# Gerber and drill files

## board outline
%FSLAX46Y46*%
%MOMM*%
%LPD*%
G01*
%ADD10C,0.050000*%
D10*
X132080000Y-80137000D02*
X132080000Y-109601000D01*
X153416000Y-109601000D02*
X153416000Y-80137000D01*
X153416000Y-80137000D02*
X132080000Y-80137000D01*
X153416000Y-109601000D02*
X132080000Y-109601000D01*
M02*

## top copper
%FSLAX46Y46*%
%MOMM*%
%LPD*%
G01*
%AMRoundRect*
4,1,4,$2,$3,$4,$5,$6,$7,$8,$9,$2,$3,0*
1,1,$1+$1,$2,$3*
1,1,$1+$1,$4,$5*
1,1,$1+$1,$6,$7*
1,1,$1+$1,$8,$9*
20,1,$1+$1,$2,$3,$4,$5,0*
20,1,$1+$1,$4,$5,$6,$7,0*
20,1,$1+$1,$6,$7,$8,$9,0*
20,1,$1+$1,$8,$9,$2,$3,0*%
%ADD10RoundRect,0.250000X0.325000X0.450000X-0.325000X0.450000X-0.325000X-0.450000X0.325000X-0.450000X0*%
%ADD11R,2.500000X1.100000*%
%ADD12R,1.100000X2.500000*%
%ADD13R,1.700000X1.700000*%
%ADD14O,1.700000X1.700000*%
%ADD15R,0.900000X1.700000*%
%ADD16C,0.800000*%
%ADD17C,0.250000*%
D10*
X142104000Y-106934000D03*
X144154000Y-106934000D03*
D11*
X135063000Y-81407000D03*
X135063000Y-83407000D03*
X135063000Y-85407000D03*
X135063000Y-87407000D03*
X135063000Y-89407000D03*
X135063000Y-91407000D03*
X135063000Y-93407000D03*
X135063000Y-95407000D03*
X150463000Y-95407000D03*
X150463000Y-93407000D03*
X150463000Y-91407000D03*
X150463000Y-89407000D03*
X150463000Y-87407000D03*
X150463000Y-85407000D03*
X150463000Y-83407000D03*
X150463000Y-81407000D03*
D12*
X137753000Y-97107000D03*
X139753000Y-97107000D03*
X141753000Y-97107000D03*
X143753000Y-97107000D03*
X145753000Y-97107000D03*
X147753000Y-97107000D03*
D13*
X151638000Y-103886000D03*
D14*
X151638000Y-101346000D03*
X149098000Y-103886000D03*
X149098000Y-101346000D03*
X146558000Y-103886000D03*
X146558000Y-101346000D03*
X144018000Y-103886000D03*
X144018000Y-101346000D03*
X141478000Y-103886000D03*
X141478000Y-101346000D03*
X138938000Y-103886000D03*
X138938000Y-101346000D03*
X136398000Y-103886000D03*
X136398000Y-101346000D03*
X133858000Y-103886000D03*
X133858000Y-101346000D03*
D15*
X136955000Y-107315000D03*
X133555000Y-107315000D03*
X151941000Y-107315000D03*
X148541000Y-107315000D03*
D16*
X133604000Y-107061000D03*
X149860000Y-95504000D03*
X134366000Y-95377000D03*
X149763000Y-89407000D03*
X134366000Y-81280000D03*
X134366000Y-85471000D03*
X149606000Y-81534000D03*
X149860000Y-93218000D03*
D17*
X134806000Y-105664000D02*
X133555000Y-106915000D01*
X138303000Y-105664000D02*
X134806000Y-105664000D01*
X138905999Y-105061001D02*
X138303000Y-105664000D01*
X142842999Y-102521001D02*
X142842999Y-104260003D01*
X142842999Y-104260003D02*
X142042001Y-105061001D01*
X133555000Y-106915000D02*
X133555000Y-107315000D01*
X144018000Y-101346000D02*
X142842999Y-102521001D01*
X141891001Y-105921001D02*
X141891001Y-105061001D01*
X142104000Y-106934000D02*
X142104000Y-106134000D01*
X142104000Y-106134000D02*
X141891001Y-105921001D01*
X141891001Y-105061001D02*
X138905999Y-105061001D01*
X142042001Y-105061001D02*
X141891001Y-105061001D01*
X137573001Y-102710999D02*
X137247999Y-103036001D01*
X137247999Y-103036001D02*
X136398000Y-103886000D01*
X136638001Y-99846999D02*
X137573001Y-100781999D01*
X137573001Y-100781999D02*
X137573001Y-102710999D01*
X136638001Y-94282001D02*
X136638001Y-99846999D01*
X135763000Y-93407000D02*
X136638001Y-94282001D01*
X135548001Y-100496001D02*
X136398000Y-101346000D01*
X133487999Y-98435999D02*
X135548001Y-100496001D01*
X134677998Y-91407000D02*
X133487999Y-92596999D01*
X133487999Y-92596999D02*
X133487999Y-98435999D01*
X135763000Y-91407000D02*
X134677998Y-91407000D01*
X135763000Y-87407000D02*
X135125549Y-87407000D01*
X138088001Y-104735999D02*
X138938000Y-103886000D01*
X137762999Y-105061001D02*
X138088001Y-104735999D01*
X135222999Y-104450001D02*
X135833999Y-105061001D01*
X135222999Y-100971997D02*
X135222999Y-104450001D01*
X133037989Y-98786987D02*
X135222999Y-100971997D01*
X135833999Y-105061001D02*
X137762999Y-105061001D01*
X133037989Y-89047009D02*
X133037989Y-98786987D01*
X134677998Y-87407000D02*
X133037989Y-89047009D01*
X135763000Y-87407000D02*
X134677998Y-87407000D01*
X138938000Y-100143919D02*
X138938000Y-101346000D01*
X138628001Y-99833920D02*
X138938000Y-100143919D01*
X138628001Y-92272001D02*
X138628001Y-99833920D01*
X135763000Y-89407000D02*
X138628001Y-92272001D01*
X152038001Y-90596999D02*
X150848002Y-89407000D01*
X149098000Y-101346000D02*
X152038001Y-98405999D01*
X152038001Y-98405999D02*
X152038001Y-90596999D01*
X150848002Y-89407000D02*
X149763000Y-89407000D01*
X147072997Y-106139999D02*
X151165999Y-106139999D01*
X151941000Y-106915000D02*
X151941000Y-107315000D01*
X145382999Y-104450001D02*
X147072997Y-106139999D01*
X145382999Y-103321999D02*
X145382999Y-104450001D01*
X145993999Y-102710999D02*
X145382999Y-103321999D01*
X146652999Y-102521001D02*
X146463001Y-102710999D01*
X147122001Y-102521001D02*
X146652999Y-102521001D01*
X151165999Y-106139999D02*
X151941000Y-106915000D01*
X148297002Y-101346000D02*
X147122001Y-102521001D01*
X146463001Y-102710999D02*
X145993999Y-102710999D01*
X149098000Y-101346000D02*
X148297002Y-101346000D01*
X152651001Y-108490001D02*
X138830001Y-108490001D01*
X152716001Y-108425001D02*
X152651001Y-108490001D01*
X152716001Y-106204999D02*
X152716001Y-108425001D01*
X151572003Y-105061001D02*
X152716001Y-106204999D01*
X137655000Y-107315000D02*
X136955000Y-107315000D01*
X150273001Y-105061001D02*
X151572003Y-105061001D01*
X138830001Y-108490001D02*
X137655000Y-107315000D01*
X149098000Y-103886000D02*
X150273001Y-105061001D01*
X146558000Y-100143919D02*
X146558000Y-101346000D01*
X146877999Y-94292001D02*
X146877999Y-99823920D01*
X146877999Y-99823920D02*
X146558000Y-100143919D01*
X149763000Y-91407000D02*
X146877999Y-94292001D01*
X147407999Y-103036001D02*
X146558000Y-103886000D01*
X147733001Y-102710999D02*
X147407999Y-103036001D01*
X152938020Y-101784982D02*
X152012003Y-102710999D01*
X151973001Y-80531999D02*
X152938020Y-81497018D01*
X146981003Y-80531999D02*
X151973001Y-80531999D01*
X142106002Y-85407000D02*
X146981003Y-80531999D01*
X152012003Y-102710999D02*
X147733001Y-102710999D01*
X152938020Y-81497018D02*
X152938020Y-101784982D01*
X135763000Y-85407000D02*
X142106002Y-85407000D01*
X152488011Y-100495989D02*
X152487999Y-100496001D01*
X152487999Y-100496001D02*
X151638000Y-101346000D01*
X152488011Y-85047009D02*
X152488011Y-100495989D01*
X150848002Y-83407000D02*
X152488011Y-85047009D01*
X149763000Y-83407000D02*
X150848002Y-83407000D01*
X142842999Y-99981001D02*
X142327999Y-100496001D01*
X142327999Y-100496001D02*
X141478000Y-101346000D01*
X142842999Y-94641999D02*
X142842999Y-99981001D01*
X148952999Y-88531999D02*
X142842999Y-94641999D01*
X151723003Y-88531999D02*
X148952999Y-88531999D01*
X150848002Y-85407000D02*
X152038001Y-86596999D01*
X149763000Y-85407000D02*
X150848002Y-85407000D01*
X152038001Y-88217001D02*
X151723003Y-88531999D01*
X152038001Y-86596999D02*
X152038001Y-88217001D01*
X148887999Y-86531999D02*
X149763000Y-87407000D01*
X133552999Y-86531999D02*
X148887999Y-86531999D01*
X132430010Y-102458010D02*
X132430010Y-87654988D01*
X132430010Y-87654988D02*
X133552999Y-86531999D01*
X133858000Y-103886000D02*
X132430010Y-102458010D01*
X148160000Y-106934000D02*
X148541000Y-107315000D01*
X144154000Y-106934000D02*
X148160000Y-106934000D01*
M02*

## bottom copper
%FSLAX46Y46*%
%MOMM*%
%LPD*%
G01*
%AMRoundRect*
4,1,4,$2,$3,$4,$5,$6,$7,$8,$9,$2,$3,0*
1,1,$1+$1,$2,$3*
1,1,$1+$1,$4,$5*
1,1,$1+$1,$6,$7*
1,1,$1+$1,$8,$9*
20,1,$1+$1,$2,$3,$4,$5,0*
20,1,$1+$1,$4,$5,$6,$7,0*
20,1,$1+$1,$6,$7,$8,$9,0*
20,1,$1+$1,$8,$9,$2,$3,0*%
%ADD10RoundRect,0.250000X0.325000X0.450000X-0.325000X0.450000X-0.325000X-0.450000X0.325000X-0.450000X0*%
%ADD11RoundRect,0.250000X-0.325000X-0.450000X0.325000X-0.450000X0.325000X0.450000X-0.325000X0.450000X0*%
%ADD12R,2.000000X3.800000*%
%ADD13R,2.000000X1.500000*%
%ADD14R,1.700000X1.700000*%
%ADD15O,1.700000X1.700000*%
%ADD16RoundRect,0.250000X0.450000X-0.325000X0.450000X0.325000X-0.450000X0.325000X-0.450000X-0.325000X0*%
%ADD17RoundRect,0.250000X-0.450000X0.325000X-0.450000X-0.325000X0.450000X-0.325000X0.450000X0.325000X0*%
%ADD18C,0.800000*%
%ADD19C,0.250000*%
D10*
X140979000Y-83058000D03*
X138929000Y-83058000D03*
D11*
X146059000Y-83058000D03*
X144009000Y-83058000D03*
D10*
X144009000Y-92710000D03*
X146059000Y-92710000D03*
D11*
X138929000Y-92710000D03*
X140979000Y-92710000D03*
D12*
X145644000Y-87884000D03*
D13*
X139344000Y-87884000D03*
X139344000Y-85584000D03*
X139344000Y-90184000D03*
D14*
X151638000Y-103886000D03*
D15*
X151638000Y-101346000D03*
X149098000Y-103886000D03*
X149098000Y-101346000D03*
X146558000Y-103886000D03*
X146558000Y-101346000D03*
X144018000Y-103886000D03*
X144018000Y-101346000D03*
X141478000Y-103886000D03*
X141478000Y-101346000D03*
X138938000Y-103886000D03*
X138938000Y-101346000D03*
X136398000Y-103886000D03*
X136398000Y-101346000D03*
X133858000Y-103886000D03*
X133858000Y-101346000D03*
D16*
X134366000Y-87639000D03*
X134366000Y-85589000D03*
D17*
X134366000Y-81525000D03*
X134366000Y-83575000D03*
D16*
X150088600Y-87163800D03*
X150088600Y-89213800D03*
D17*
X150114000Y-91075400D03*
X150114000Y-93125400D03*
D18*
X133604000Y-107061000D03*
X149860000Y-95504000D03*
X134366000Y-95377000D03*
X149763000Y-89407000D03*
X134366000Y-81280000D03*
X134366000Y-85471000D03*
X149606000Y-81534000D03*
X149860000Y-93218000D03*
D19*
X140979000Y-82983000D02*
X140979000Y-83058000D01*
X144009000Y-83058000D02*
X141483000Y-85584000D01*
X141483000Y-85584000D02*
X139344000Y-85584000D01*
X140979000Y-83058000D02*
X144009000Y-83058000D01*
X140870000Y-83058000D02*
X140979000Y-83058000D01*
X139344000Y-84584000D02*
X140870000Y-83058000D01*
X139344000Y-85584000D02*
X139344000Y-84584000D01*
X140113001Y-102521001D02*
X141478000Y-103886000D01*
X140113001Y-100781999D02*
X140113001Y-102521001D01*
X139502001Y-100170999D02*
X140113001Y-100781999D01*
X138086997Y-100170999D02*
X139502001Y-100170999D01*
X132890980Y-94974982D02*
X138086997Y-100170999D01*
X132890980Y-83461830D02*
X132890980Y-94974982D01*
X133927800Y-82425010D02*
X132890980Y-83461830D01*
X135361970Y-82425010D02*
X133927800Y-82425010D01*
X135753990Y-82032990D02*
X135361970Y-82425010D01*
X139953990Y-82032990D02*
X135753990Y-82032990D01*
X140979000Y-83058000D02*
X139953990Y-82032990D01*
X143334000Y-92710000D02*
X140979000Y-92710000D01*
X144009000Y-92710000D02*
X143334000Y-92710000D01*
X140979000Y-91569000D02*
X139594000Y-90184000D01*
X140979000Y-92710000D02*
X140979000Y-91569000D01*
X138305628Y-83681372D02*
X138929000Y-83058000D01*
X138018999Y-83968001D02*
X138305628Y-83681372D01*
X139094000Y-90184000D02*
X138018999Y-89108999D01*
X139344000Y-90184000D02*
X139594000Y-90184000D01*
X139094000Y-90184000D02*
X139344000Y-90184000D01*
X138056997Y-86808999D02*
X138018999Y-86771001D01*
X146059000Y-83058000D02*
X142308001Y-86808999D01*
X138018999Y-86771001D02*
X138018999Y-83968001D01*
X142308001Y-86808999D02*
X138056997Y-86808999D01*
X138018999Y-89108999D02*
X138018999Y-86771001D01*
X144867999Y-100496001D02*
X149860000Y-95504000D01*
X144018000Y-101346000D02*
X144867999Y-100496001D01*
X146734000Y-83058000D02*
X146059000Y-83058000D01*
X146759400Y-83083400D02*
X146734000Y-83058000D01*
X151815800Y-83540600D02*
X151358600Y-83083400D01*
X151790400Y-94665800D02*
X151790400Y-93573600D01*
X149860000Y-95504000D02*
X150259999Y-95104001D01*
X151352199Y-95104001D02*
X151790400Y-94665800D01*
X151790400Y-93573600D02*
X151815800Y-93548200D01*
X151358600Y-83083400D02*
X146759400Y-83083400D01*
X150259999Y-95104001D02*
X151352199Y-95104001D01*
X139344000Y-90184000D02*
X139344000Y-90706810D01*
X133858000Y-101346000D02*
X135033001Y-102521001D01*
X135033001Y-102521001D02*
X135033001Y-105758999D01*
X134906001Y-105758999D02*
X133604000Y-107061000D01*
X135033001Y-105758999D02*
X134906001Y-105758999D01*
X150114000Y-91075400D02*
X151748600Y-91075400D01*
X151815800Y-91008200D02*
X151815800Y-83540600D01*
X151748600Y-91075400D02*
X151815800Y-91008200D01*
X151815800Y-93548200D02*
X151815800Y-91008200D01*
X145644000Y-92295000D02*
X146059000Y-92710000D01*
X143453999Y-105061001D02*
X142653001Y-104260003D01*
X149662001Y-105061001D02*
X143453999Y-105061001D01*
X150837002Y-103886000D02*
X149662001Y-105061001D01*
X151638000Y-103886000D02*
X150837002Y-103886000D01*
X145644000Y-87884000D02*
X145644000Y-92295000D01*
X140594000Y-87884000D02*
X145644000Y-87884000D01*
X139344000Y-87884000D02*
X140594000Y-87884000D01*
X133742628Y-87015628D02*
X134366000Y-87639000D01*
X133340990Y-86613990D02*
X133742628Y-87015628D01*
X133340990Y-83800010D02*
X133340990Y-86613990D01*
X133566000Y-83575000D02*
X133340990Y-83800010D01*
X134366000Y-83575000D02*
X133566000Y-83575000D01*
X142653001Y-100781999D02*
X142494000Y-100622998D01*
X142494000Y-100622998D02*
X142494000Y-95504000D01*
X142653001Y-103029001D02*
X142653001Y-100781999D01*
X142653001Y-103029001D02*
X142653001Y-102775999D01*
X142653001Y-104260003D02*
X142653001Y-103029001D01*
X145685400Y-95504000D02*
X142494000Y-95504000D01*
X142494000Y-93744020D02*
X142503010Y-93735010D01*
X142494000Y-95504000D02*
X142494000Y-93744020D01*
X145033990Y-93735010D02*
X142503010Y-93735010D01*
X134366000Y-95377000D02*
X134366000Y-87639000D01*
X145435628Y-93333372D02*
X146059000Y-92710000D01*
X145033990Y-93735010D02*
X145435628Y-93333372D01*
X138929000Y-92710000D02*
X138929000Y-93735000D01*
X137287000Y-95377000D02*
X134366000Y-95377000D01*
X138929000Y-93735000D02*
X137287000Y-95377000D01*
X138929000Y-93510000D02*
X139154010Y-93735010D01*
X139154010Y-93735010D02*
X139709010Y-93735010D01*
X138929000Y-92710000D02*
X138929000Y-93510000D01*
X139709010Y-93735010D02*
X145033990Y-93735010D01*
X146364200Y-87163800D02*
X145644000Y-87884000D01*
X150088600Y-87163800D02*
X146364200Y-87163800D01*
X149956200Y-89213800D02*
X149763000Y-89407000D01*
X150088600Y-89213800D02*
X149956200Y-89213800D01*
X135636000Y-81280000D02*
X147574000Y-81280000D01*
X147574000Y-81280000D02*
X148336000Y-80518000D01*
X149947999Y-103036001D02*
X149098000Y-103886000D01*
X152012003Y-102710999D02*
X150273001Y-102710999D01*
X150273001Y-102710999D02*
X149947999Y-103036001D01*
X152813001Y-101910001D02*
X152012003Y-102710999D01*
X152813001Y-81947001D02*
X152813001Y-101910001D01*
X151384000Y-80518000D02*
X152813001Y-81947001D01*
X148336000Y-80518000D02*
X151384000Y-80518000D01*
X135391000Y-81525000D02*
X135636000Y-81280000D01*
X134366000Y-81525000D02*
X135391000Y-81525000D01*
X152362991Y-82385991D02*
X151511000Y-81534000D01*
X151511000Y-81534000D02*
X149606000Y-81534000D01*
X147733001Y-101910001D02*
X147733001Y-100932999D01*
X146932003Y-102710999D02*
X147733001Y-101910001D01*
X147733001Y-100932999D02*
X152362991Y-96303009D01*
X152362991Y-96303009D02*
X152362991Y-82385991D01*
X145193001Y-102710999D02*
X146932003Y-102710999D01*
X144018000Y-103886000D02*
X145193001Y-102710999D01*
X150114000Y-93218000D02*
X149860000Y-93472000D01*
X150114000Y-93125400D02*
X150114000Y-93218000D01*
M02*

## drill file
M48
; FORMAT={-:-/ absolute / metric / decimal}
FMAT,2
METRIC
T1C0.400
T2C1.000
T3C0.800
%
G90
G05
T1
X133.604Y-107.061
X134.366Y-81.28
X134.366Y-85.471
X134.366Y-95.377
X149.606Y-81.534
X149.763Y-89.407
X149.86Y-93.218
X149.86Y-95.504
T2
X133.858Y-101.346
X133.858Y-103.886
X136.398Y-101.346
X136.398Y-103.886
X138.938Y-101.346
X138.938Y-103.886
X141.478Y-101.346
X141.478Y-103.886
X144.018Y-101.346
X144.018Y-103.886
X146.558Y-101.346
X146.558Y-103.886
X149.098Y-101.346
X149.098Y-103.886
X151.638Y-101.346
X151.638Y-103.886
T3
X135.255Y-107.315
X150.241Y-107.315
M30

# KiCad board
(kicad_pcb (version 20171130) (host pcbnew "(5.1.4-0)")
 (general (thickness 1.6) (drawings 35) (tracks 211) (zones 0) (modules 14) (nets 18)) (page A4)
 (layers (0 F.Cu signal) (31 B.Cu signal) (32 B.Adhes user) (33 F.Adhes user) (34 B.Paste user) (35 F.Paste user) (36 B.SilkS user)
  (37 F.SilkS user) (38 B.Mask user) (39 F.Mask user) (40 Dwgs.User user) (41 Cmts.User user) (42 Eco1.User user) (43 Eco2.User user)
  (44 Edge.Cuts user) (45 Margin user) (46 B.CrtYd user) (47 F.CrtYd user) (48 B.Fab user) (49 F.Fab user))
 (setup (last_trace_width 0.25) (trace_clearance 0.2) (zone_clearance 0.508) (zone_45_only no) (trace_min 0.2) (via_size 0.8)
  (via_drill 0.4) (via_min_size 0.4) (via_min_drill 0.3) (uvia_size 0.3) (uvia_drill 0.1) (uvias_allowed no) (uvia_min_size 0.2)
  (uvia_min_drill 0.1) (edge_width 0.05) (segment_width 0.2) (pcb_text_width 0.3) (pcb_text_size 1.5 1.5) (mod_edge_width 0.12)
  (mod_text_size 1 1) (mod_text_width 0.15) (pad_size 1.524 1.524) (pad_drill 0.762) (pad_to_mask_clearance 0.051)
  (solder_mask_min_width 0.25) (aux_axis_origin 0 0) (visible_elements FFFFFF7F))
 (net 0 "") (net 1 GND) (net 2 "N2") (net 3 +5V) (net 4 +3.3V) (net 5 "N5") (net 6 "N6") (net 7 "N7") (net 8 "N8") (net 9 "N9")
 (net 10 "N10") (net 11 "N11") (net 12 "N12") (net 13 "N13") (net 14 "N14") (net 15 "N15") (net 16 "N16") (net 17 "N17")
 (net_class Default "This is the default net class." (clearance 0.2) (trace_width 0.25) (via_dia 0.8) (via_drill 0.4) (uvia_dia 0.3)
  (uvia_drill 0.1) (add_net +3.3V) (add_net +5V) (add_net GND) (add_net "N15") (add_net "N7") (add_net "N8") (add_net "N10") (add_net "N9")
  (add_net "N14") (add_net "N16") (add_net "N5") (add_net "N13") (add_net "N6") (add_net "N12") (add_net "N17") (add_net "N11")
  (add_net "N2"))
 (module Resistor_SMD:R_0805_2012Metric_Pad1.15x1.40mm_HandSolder (layer F.Cu) (at 143.129 106.934 180)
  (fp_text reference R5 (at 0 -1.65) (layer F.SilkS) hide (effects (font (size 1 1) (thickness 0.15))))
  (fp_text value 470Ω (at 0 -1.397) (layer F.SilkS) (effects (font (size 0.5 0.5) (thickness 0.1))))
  (pad 2 smd roundrect (at 1.025 0 180) (size 1.15 1.4) (layers F.Cu F.Paste F.Mask) (roundrect_rratio 0.217391) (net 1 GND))
  (pad 1 smd roundrect (at -1.025 0 180) (size 1.15 1.4) (layers F.Cu F.Paste F.Mask) (roundrect_rratio 0.217391) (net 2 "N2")))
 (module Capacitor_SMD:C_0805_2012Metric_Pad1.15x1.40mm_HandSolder (layer B.Cu) (at 139.954 83.058 180)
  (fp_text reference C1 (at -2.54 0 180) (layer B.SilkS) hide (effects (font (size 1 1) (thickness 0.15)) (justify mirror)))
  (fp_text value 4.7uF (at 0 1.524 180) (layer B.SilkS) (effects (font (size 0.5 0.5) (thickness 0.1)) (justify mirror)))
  (pad 1 smd roundrect (at -1.025 0 180) (size 1.15 1.4) (layers B.Cu B.Paste B.Mask) (roundrect_rratio 0.217391) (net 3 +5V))
  (pad 2 smd roundrect (at 1.025 0 180) (size 1.15 1.4) (layers B.Cu B.Paste B.Mask) (roundrect_rratio 0.217391) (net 1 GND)))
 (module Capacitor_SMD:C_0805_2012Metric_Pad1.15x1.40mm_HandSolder (layer B.Cu) (at 145.034 83.058)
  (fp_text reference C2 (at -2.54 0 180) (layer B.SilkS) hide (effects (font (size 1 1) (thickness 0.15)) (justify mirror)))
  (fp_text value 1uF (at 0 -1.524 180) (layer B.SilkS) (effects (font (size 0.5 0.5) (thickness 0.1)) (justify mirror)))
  (pad 2 smd roundrect (at 1.025 0) (size 1.15 1.4) (layers B.Cu B.Paste B.Mask) (roundrect_rratio 0.217391) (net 1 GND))
  (pad 1 smd roundrect (at -1.025 0) (size 1.15 1.4) (layers B.Cu B.Paste B.Mask) (roundrect_rratio 0.217391) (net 3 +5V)))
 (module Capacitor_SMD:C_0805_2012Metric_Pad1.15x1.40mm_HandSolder (layer B.Cu) (at 145.034 92.71 180)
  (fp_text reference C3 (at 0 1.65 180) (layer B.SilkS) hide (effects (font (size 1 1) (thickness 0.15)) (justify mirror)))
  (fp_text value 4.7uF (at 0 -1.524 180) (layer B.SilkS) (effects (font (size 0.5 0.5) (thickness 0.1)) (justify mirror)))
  (pad 2 smd roundrect (at 1.025 0 180) (size 1.15 1.4) (layers B.Cu B.Paste B.Mask) (roundrect_rratio 0.217391) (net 1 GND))
  (pad 1 smd roundrect (at -1.025 0 180) (size 1.15 1.4) (layers B.Cu B.Paste B.Mask) (roundrect_rratio 0.217391) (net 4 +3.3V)))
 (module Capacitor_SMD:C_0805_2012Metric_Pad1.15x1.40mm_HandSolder (layer B.Cu) (at 139.954 92.71)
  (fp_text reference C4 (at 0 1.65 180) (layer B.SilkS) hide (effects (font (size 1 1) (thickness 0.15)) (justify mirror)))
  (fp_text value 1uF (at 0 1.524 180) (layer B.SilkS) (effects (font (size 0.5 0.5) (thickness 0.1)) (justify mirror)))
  (pad 1 smd roundrect (at -1.025 0) (size 1.15 1.4) (layers B.Cu B.Paste B.Mask) (roundrect_rratio 0.217391) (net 4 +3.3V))
  (pad 2 smd roundrect (at 1.025 0) (size 1.15 1.4) (layers B.Cu B.Paste B.Mask) (roundrect_rratio 0.217391) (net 1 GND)))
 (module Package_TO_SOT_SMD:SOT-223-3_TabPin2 (layer B.Cu) (at 142.494 87.884)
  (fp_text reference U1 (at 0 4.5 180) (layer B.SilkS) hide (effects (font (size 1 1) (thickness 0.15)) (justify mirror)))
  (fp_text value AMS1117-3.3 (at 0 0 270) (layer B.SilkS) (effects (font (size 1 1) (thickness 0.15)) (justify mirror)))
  (pad 2 smd rect (at 3.15 0) (size 2 3.8) (layers B.Cu B.Paste B.Mask) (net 4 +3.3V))
  (pad 2 smd rect (at -3.15 0) (size 2 1.5) (layers B.Cu B.Paste B.Mask) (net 4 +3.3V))
  (pad 3 smd rect (at -3.15 -2.3) (size 2 1.5) (layers B.Cu B.Paste B.Mask) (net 3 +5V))
  (pad 1 smd rect (at -3.15 2.3) (size 2 1.5) (layers B.Cu B.Paste B.Mask) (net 1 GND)))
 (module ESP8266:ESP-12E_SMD (layer F.Cu) (at 135.763 81.407)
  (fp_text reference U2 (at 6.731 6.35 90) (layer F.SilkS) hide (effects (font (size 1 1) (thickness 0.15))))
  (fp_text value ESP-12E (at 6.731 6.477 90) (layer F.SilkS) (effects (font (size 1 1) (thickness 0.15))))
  (pad 1 smd rect (at 0 0) (size 2.5 1.1) (drill (offset -0.7 0)) (layers F.Cu F.Paste F.Mask) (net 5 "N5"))
  (pad 2 smd rect (at 0 2) (size 2.5 1.1) (drill (offset -0.7 0)) (layers F.Cu F.Paste F.Mask))
  (pad 3 smd rect (at 0 4) (size 2.5 1.1) (drill (offset -0.7 0)) (layers F.Cu F.Paste F.Mask) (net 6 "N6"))
  (pad 4 smd rect (at 0 6) (size 2.5 1.1) (drill (offset -0.7 0)) (layers F.Cu F.Paste F.Mask) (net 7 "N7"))
  (pad 5 smd rect (at 0 8) (size 2.5 1.1) (drill (offset -0.7 0)) (layers F.Cu F.Paste F.Mask) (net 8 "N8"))
  (pad 6 smd rect (at 0 10) (size 2.5 1.1) (drill (offset -0.7 0)) (layers F.Cu F.Paste F.Mask) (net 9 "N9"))
  (pad 7 smd rect (at 0 12) (size 2.5 1.1) (drill (offset -0.7 0)) (layers F.Cu F.Paste F.Mask) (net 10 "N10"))
  (pad 8 smd rect (at 0 14) (size 2.5 1.1) (drill (offset -0.7 0)) (layers F.Cu F.Paste F.Mask) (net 4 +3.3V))
  (pad 9 smd rect (at 14 14) (size 2.5 1.1) (drill (offset 0.7 0)) (layers F.Cu F.Paste F.Mask) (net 1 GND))
  (pad 10 smd rect (at 14 12) (size 2.5 1.1) (drill (offset 0.7 0)) (layers F.Cu F.Paste F.Mask) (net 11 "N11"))
  (pad 11 smd rect (at 14 10) (size 2.5 1.1) (drill (offset 0.7 0)) (layers F.Cu F.Paste F.Mask) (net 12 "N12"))
  (pad 12 smd rect (at 14 8) (size 2.5 1.1) (drill (offset 0.7 0)) (layers F.Cu F.Paste F.Mask) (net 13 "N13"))
  (pad 13 smd rect (at 14 6) (size 2.5 1.1) (drill (offset 0.7 0)) (layers F.Cu F.Paste F.Mask) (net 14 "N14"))
  (pad 14 smd rect (at 14 4) (size 2.5 1.1) (drill (offset 0.7 0)) (layers F.Cu F.Paste F.Mask) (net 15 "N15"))
  (pad 15 smd rect (at 14 2) (size 2.5 1.1) (drill (offset 0.7 0)) (layers F.Cu F.Paste F.Mask) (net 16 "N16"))
  (pad 16 smd rect (at 14 0) (size 2.5 1.1) (drill (offset 0.7 0)) (layers F.Cu F.Paste F.Mask) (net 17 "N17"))
  (pad 17 smd rect (at 1.99 15 90) (size 2.5 1.1) (drill (offset -0.7 0)) (layers F.Cu F.Paste F.Mask))
  (pad 18 smd rect (at 3.99 15 90) (size 2.5 1.1) (drill (offset -0.7 0)) (layers F.Cu F.Paste F.Mask))
  (pad 19 smd rect (at 5.99 15 90) (size 2.5 1.1) (drill (offset -0.7 0)) (layers F.Cu F.Paste F.Mask))
  (pad 20 smd rect (at 7.99 15 90) (size 2.5 1.1) (drill (offset -0.7 0)) (layers F.Cu F.Paste F.Mask))
  (pad 21 smd rect (at 9.99 15 90) (size 2.5 1.1) (drill (offset -0.7 0)) (layers F.Cu F.Paste F.Mask))
  (pad 22 smd rect (at 11.99 15 90) (size 2.5 1.1) (drill (offset -0.7 0)) (layers F.Cu F.Paste F.Mask)))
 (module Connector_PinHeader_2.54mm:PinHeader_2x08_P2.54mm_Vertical (layer B.Cu) (at 151.638 103.886 90)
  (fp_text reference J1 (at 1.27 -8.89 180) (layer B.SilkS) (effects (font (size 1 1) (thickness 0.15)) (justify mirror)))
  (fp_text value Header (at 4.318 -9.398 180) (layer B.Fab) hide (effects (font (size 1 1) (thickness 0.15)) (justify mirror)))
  (pad 1 thru_hole rect (at 0 0 90) (size 1.7 1.7) (drill 1) (layers *.Cu *.Mask) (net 4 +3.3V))
  (pad 2 thru_hole oval (at 2.54 0 90) (size 1.7 1.7) (drill 1) (layers *.Cu *.Mask) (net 16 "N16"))
  (pad 3 thru_hole oval (at 0 -2.54 90) (size 1.7 1.7) (drill 1) (layers *.Cu *.Mask) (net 5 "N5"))
  (pad 4 thru_hole oval (at 2.54 -2.54 90) (size 1.7 1.7) (drill 1) (layers *.Cu *.Mask) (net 13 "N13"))
  (pad 5 thru_hole oval (at 0 -5.08 90) (size 1.7 1.7) (drill 1) (layers *.Cu *.Mask) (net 6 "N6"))
  (pad 6 thru_hole oval (at 2.54 -5.08 90) (size 1.7 1.7) (drill 1) (layers *.Cu *.Mask) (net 12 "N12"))
  (pad 7 thru_hole oval (at 0 -7.62 90) (size 1.7 1.7) (drill 1) (layers *.Cu *.Mask) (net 17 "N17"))
  (pad 8 thru_hole oval (at 2.54 -7.62 90) (size 1.7 1.7) (drill 1) (layers *.Cu *.Mask) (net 1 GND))
  (pad 9 thru_hole oval (at 0 -10.16 90) (size 1.7 1.7) (drill 1) (layers *.Cu *.Mask) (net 3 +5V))
  (pad 10 thru_hole oval (at 2.54 -10.16 90) (size 1.7 1.7) (drill 1) (layers *.Cu *.Mask) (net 15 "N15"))
  (pad 11 thru_hole oval (at 0 -12.7 90) (size 1.7 1.7) (drill 1) (layers *.Cu *.Mask) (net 7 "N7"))
  (pad 12 thru_hole oval (at 2.54 -12.7 90) (size 1.7 1.7) (drill 1) (layers *.Cu *.Mask) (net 8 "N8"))
  (pad 13 thru_hole oval (at 0 -15.24 90) (size 1.7 1.7) (drill 1) (layers *.Cu *.Mask) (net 10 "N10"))
  (pad 14 thru_hole oval (at 2.54 -15.24 90) (size 1.7 1.7) (drill 1) (layers *.Cu *.Mask) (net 9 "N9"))
  (pad 15 thru_hole oval (at 0 -17.78 90) (size 1.7 1.7) (drill 1) (layers *.Cu *.Mask) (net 14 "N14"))
  (pad 16 thru_hole oval (at 2.54 -17.78 90) (size 1.7 1.7) (drill 1) (layers *.Cu *.Mask) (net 1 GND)))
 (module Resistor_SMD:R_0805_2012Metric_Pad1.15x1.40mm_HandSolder (layer B.Cu) (at 134.366 86.614 90)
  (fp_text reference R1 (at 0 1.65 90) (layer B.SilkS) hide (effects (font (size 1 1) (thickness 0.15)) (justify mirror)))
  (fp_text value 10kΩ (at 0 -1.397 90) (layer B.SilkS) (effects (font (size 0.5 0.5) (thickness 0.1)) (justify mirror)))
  (pad 1 smd roundrect (at -1.025 0 90) (size 1.15 1.4) (layers B.Cu B.Paste B.Mask) (roundrect_rratio 0.217391) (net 4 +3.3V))
  (pad 2 smd roundrect (at 1.025 0 90) (size 1.15 1.4) (layers B.Cu B.Paste B.Mask) (roundrect_rratio 0.217391) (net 6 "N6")))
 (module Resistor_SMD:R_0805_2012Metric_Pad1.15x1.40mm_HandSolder (layer B.Cu) (at 134.366 82.55 270)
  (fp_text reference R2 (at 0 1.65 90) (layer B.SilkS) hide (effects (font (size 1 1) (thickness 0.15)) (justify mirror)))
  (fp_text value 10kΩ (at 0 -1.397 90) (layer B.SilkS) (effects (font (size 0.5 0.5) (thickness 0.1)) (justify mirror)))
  (pad 1 smd roundrect (at -1.025 0 270) (size 1.15 1.4) (layers B.Cu B.Paste B.Mask) (roundrect_rratio 0.217391) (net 5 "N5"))
  (pad 2 smd roundrect (at 1.025 0 270) (size 1.15 1.4) (layers B.Cu B.Paste B.Mask) (roundrect_rratio 0.217391) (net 4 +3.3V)))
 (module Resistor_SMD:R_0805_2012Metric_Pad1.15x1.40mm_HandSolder (layer B.Cu) (at 150.0886 88.1888 90)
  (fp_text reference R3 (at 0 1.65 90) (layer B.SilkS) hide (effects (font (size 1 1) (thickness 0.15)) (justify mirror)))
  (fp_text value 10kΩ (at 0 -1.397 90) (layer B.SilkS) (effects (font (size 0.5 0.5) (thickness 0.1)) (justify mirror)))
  (pad 2 smd roundrect (at 1.025 0 90) (size 1.15 1.4) (layers B.Cu B.Paste B.Mask) (roundrect_rratio 0.217391) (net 4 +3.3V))
  (pad 1 smd roundrect (at -1.025 0 90) (size 1.15 1.4) (layers B.Cu B.Paste B.Mask) (roundrect_rratio 0.217391) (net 13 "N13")))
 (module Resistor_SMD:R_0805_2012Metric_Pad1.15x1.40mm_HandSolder (layer B.Cu) (at 150.114 92.1004 270)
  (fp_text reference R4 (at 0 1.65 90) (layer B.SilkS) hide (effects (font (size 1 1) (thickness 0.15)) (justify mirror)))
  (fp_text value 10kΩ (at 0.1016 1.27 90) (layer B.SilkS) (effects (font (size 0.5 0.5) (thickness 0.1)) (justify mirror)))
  (pad 1 smd roundrect (at -1.025 0 270) (size 1.15 1.4) (layers B.Cu B.Paste B.Mask) (roundrect_rratio 0.217391) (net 1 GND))
  (pad 2 smd roundrect (at 1.025 0 270) (size 1.15 1.4) (layers B.Cu B.Paste B.Mask) (roundrect_rratio 0.217391) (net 11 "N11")))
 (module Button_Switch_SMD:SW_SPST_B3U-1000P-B (layer F.Cu) (at 135.255 107.315)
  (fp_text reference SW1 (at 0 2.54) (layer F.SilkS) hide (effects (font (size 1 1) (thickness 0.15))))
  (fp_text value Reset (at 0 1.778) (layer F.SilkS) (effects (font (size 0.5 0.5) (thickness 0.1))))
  (pad "" np_thru_hole circle (at 0 0) (size 0.8 0.8) (drill 0.8) (layers *.Cu *.Mask))
  (pad 2 smd rect (at 1.7 0) (size 0.9 1.7) (layers F.Cu F.Paste F.Mask) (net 5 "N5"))
  (pad 1 smd rect (at -1.7 0) (size 0.9 1.7) (layers F.Cu F.Paste F.Mask) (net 1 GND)))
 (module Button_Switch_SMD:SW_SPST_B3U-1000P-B (layer F.Cu) (at 150.241 107.315 180)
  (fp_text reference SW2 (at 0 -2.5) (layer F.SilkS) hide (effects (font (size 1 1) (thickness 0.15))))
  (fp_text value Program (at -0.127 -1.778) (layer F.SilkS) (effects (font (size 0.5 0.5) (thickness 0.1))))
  (pad 1 smd rect (at -1.7 0 180) (size 0.9 1.7) (layers F.Cu F.Paste F.Mask) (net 13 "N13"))
  (pad 2 smd rect (at 1.7 0 180) (size 0.9 1.7) (layers F.Cu F.Paste F.Mask) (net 2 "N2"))
  (pad "" np_thru_hole circle (at 0 0 180) (size 0.8 0.8) (drill 0.8) (layers *.Cu *.Mask)))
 (gr_line (start 132.08 80.137) (end 132.08 109.601) (layer Edge.Cuts) (width 0.05))
 (gr_line (start 153.416 109.601) (end 153.416 80.137) (layer Edge.Cuts) (width 0.05))
 (gr_line (start 153.416 80.137) (end 132.08 80.137) (layer Edge.Cuts) (width 0.05))
 (gr_line (start 153.416 109.601) (end 132.08 109.601) (layer Edge.Cuts) (width 0.05))
 (segment (start 140.979 82.983) (end 140.979 83.058) (width 0.25) (layer B.Cu) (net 3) (status 30))
 (segment (start 144.009 83.058) (end 141.483 85.584) (width 0.25) (layer B.Cu) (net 3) (status 10))
 (segment (start 141.483 85.584) (end 139.344 85.584) (width 0.25) (layer B.Cu) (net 3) (status 20))
 (segment (start 140.979 83.058) (end 144.009 83.058) (width 0.25) (layer B.Cu) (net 3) (status 30))
 (segment (start 140.87 83.058) (end 140.979 83.058) (width 0.25) (layer B.Cu) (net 3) (status 30))
 (segment (start 139.344 84.584) (end 140.87 83.058) (width 0.25) (layer B.Cu) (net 3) (status 20))
 (segment (start 139.344 85.584) (end 139.344 84.584) (width 0.25) (layer B.Cu) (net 3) (status 10))
 (segment (start 140.113001 102.521001) (end 141.478 103.886) (width 0.25) (layer B.Cu) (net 3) (status 20))
 (segment (start 140.113001 100.781999) (end 140.113001 102.521001) (width 0.25) (layer B.Cu) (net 3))
 (segment (start 139.502001 100.170999) (end 140.113001 100.781999) (width 0.25) (layer B.Cu) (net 3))
 (segment (start 138.086997 100.170999) (end 139.502001 100.170999) (width 0.25) (layer B.Cu) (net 3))
 (segment (start 132.89098 94.974982) (end 138.086997 100.170999) (width 0.25) (layer B.Cu) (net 3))
 (segment (start 132.89098 83.46183) (end 132.89098 94.974982) (width 0.25) (layer B.Cu) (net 3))
 (segment (start 133.9278 82.42501) (end 132.89098 83.46183) (width 0.25) (layer B.Cu) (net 3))
 (segment (start 135.36197 82.42501) (end 133.9278 82.42501) (width 0.25) (layer B.Cu) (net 3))
 (segment (start 135.75399 82.03299) (end 135.36197 82.42501) (width 0.25) (layer B.Cu) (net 3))
 (segment (start 139.95399 82.03299) (end 135.75399 82.03299) (width 0.25) (layer B.Cu) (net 3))
 (segment (start 140.979 83.058) (end 139.95399 82.03299) (width 0.25) (layer B.Cu) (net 3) (status 10))
 (via (at 133.604 107.061) (size 0.8) (drill 0.4) (layers F.Cu B.Cu) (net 1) (status 30))
 (via (at 149.86 95.504) (size 0.8) (drill 0.4) (layers F.Cu B.Cu) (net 1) (status 30))
 (segment (start 143.334 92.71) (end 140.979 92.71) (width 0.25) (layer B.Cu) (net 1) (status 20))
 (segment (start 144.009 92.71) (end 143.334 92.71) (width 0.25) (layer B.Cu) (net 1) (status 10))
 (segment (start 140.979 91.569) (end 139.594 90.184) (width 0.25) (layer B.Cu) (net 1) (status 20))
 (segment (start 140.979 92.71) (end 140.979 91.569) (width 0.25) (layer B.Cu) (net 1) (status 10))
 (segment (start 138.305628 83.681372) (end 138.929 83.058) (width 0.25) (layer B.Cu) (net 1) (status 20))
 (segment (start 138.018999 83.968001) (end 138.305628 83.681372) (width 0.25) (layer B.Cu) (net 1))
 (segment (start 139.094 90.184) (end 138.018999 89.108999) (width 0.25) (layer B.Cu) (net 1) (status 10))
 (segment (start 139.344 90.184) (end 139.594 90.184) (width 0.25) (layer B.Cu) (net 1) (status 30))
 (segment (start 139.094 90.184) (end 139.344 90.184) (width 0.25) (layer B.Cu) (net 1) (status 30))
 (segment (start 138.056997 86.808999) (end 138.018999 86.771001) (width 0.25) (layer B.Cu) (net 1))
 (segment (start 146.059 83.058) (end 142.308001 86.808999) (width 0.25) (layer B.Cu) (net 1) (status 10))
 (segment (start 138.018999 86.771001) (end 138.018999 83.968001) (width 0.25) (layer B.Cu) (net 1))
 (segment (start 142.308001 86.808999) (end 138.056997 86.808999) (width 0.25) (layer B.Cu) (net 1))
 (segment (start 138.018999 89.108999) (end 138.018999 86.771001) (width 0.25) (layer B.Cu) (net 1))
 (segment (start 144.867999 100.496001) (end 149.86 95.504) (width 0.25) (layer B.Cu) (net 1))
 (segment (start 144.018 101.346) (end 144.867999 100.496001) (width 0.25) (layer B.Cu) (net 1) (status 10))
 (segment (start 146.734 83.058) (end 146.059 83.058) (width 0.25) (layer B.Cu) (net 1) (status 20))
 (segment (start 146.7594 83.0834) (end 146.734 83.058) (width 0.25) (layer B.Cu) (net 1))
 (segment (start 151.8158 83.5406) (end 151.3586 83.0834) (width 0.25) (layer B.Cu) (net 1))
 (segment (start 151.7904 94.6658) (end 151.7904 93.5736) (width 0.25) (layer B.Cu) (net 1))
 (segment (start 149.86 95.504) (end 150.259999 95.104001) (width 0.25) (layer B.Cu) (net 1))
 (segment (start 151.352199 95.104001) (end 151.7904 94.6658) (width 0.25) (layer B.Cu) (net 1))
 (segment (start 151.7904 93.5736) (end 151.8158 93.5482) (width 0.25) (layer B.Cu) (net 1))
 (segment (start 151.3586 83.0834) (end 146.7594 83.0834) (width 0.25) (layer B.Cu) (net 1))
 (segment (start 150.259999 95.104001) (end 151.352199 95.104001) (width 0.25) (layer B.Cu) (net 1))
 (segment (start 139.344 90.184) (end 139.344 90.70681) (width 0.25) (layer B.Cu) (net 1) (status 30))
 (segment (start 133.858 101.346) (end 135.033001 102.521001) (width 0.25) (layer B.Cu) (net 1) (status 10))
 (segment (start 135.033001 102.521001) (end 135.033001 105.758999) (width 0.25) (layer B.Cu) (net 1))
 (segment (start 134.906001 105.758999) (end 133.604 107.061) (width 0.25) (layer B.Cu) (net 1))
 (segment (start 135.033001 105.758999) (end 134.906001 105.758999) (width 0.25) (layer B.Cu) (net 1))
 (segment (start 134.806 105.664) (end 133.555 106.915) (width 0.25) (layer F.Cu) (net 1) (status 20))
 (segment (start 138.303 105.664) (end 134.806 105.664) (width 0.25) (layer F.Cu) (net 1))
 (segment (start 138.905999 105.061001) (end 138.303 105.664) (width 0.25) (layer F.Cu) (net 1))
 (segment (start 142.842999 102.521001) (end 142.842999 104.260003) (width 0.25) (layer F.Cu) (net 1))
 (segment (start 142.842999 104.260003) (end 142.042001 105.061001) (width 0.25) (layer F.Cu) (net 1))
 (segment (start 133.555 106.915) (end 133.555 107.315) (width 0.25) (layer F.Cu) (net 1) (status 30))
 (segment (start 144.018 101.346) (end 142.842999 102.521001) (width 0.25) (layer F.Cu) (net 1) (status 10))
 (segment (start 141.891001 105.921001) (end 141.891001 105.061001) (width 0.25) (layer F.Cu) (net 1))
 (segment (start 142.104 106.934) (end 142.104 106.134) (width 0.25) (layer F.Cu) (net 1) (status 10))
 (segment (start 142.104 106.134) (end 141.891001 105.921001) (width 0.25) (layer F.Cu) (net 1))
 (segment (start 141.891001 105.061001) (end 138.905999 105.061001) (width 0.25) (layer F.Cu) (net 1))
 (segment (start 142.042001 105.061001) (end 141.891001 105.061001) (width 0.25) (layer F.Cu) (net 1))
 (segment (start 150.114 91.0754) (end 151.7486 91.0754) (width 0.25) (layer B.Cu) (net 1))
 (segment (start 151.8158 91.0082) (end 151.8158 83.5406) (width 0.25) (layer B.Cu) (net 1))
 (segment (start 151.7486 91.0754) (end 151.8158 91.0082) (width 0.25) (layer B.Cu) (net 1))
 (segment (start 151.8158 93.5482) (end 151.8158 91.0082) (width 0.25) (layer B.Cu) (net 1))
 (via (at 134.366 95.377) (size 0.8) (drill 0.4) (layers F.Cu B.Cu) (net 4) (status 30))
 (segment (start 145.644 92.295) (end 146.059 92.71) (width 0.25) (layer B.Cu) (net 4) (status 30))
 (segment (start 143.453999 105.061001) (end 142.653001 104.260003) (width 0.25) (layer B.Cu) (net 4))
 (segment (start 149.662001 105.061001) (end 143.453999 105.061001) (width 0.25) (layer B.Cu) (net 4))
 (segment (start 150.837002 103.886) (end 149.662001 105.061001) (width 0.25) (layer B.Cu) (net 4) (status 10))
 (segment (start 151.638 103.886) (end 150.837002 103.886) (width 0.25) (layer B.Cu) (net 4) (status 30))
 (segment (start 145.644 87.884) (end 145.644 92.295) (width 0.25) (layer B.Cu) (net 4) (status 30))
 (segment (start 140.594 87.884) (end 145.644 87.884) (width 0.25) (layer B.Cu) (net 4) (status 20))
 (segment (start 139.344 87.884) (end 140.594 87.884) (width 0.25) (layer B.Cu) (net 4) (status 10))
 (segment (start 133.742628 87.015628) (end 134.366 87.639) (width 0.25) (layer B.Cu) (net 4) (status 20))
 (segment (start 133.34099 86.61399) (end 133.742628 87.015628) (width 0.25) (layer B.Cu) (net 4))
 (segment (start 133.34099 83.80001) (end 133.34099 86.61399) (width 0.25) (layer B.Cu) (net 4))
 (segment (start 133.566 83.575) (end 133.34099 83.80001) (width 0.25) (layer B.Cu) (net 4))
 (segment (start 134.366 83.575) (end 133.566 83.575) (width 0.25) (layer B.Cu) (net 4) (status 10))
 (segment (start 142.653001 100.781999) (end 142.494 100.622998) (width 0.25) (layer B.Cu) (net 4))
 (segment (start 142.494 100.622998) (end 142.494 95.504) (width 0.25) (layer B.Cu) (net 4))
 (segment (start 142.653001 103.029001) (end 142.653001 100.781999) (width 0.25) (layer B.Cu) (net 4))
 (segment (start 142.653001 103.029001) (end 142.653001 102.775999) (width 0.25) (layer B.Cu) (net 4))
 (segment (start 142.653001 104.260003) (end 142.653001 103.029001) (width 0.25) (layer B.Cu) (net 4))
 (segment (start 145.6854 95.504) (end 142.494 95.504) (width 0.25) (layer B.Cu) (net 4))
 (segment (start 142.494 93.74402) (end 142.50301 93.73501) (width 0.25) (layer B.Cu) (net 4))
 (segment (start 142.494 95.504) (end 142.494 93.74402) (width 0.25) (layer B.Cu) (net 4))
 (segment (start 145.03399 93.73501) (end 142.50301 93.73501) (width 0.25) (layer B.Cu) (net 4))
 (segment (start 134.366 95.377) (end 134.366 87.639) (width 0.25) (layer B.Cu) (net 4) (status 20))
 (segment (start 145.435628 93.333372) (end 146.059 92.71) (width 0.25) (layer B.Cu) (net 4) (status 20))
 (segment (start 145.03399 93.73501) (end 145.435628 93.333372) (width 0.25) (layer B.Cu) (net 4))
 (segment (start 138.929 92.71) (end 138.929 93.735) (width 0.25) (layer B.Cu) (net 4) (status 10))
 (segment (start 137.287 95.377) (end 134.366 95.377) (width 0.25) (layer B.Cu) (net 4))
 (segment (start 138.929 93.735) (end 137.287 95.377) (width 0.25) (layer B.Cu) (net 4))
 (segment (start 138.929 93.51) (end 139.15401 93.73501) (width 0.25) (layer B.Cu) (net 4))
 (segment (start 139.15401 93.73501) (end 139.70901 93.73501) (width 0.25) (layer B.Cu) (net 4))
 (segment (start 138.929 92.71) (end 138.929 93.51) (width 0.25) (layer B.Cu) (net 4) (status 10))
 (segment (start 139.70901 93.73501) (end 145.03399 93.73501) (width 0.25) (layer B.Cu) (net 4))
 (segment (start 146.3642 87.1638) (end 145.644 87.884) (width 0.25) (layer B.Cu) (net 4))
 (segment (start 150.0886 87.1638) (end 146.3642 87.1638) (width 0.25) (layer B.Cu) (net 4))
 (segment (start 137.573001 102.710999) (end 137.247999 103.036001) (width 0.25) (layer F.Cu) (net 10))
 (segment (start 137.247999 103.036001) (end 136.398 103.886) (width 0.25) (layer F.Cu) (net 10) (status 20))
 (segment (start 136.638001 99.846999) (end 137.573001 100.781999) (width 0.25) (layer F.Cu) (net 10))
 (segment (start 137.573001 100.781999) (end 137.573001 102.710999) (width 0.25) (layer F.Cu) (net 10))
 (segment (start 136.638001 94.282001) (end 136.638001 99.846999) (width 0.25) (layer F.Cu) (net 10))
 (segment (start 135.763 93.407) (end 136.638001 94.282001) (width 0.25) (layer F.Cu) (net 10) (status 10))
 (segment (start 135.548001 100.496001) (end 136.398 101.346) (width 0.25) (layer F.Cu) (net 9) (status 20))
 (segment (start 133.487999 98.435999) (end 135.548001 100.496001) (width 0.25) (layer F.Cu) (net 9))
 (segment (start 134.677998 91.407) (end 133.487999 92.596999) (width 0.25) (layer F.Cu) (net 9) (status 10))
 (segment (start 133.487999 92.596999) (end 133.487999 98.435999) (width 0.25) (layer F.Cu) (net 9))
 (segment (start 135.763 91.407) (end 134.677998 91.407) (width 0.25) (layer F.Cu) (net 9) (status 30))
 (segment (start 135.763 87.407) (end 135.125549 87.407) (width 0.25) (layer F.Cu) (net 7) (status 30))
 (segment (start 138.088001 104.735999) (end 138.938 103.886) (width 0.25) (layer F.Cu) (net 7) (status 20))
 (segment (start 137.762999 105.061001) (end 138.088001 104.735999) (width 0.25) (layer F.Cu) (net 7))
 (segment (start 135.222999 104.450001) (end 135.833999 105.061001) (width 0.25) (layer F.Cu) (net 7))
 (segment (start 135.222999 100.971997) (end 135.222999 104.450001) (width 0.25) (layer F.Cu) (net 7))
 (segment (start 133.037989 98.786987) (end 135.222999 100.971997) (width 0.25) (layer F.Cu) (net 7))
 (segment (start 135.833999 105.061001) (end 137.762999 105.061001) (width 0.25) (layer F.Cu) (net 7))
 (segment (start 133.037989 89.047009) (end 133.037989 98.786987) (width 0.25) (layer F.Cu) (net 7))
 (segment (start 134.677998 87.407) (end 133.037989 89.047009) (width 0.25) (layer F.Cu) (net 7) (status 10))
 (segment (start 135.763 87.407) (end 134.677998 87.407) (width 0.25) (layer F.Cu) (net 7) (status 30))
 (segment (start 138.938 100.143919) (end 138.938 101.346) (width 0.25) (layer F.Cu) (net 8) (status 20))
 (segment (start 138.628001 99.83392) (end 138.938 100.143919) (width 0.25) (layer F.Cu) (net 8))
 (segment (start 138.628001 92.272001) (end 138.628001 99.83392) (width 0.25) (layer F.Cu) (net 8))
 (segment (start 135.763 89.407) (end 138.628001 92.272001) (width 0.25) (layer F.Cu) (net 8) (status 10))
 (segment (start 152.038001 90.596999) (end 150.848002 89.407) (width 0.25) (layer F.Cu) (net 13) (status 20))
 (via (at 149.763 89.407) (size 0.8) (drill 0.4) (layers F.Cu B.Cu) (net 13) (status 30))
 (segment (start 149.098 101.346) (end 152.038001 98.405999) (width 0.25) (layer F.Cu) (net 13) (status 10))
 (segment (start 152.038001 98.405999) (end 152.038001 90.596999) (width 0.25) (layer F.Cu) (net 13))
 (segment (start 150.848002 89.407) (end 149.763 89.407) (width 0.25) (layer F.Cu) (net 13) (status 30))
 (segment (start 149.9562 89.2138) (end 149.763 89.407) (width 0.25) (layer B.Cu) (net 13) (status 30))
 (segment (start 150.0886 89.2138) (end 149.9562 89.2138) (width 0.25) (layer B.Cu) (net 13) (status 30))
 (segment (start 147.072997 106.139999) (end 151.165999 106.139999) (width 0.25) (layer F.Cu) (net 13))
 (segment (start 151.941 106.915) (end 151.941 107.315) (width 0.25) (layer F.Cu) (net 13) (status 30))
 (segment (start 145.382999 104.450001) (end 147.072997 106.139999) (width 0.25) (layer F.Cu) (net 13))
 (segment (start 145.382999 103.321999) (end 145.382999 104.450001) (width 0.25) (layer F.Cu) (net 13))
 (segment (start 145.993999 102.710999) (end 145.382999 103.321999) (width 0.25) (layer F.Cu) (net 13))
 (segment (start 146.652999 102.521001) (end 146.463001 102.710999) (width 0.25) (layer F.Cu) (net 13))
 (segment (start 147.122001 102.521001) (end 146.652999 102.521001) (width 0.25) (layer F.Cu) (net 13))
 (segment (start 151.165999 106.139999) (end 151.941 106.915) (width 0.25) (layer F.Cu) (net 13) (status 20))
 (segment (start 148.297002 101.346) (end 147.122001 102.521001) (width 0.25) (layer F.Cu) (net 13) (status 10))
 (segment (start 146.463001 102.710999) (end 145.993999 102.710999) (width 0.25) (layer F.Cu) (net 13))
 (segment (start 149.098 101.346) (end 148.297002 101.346) (width 0.25) (layer F.Cu) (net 13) (status 30))
 (via (at 134.366 81.28) (size 0.8) (drill 0.4) (layers F.Cu B.Cu) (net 5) (status 30))
 (segment (start 135.636 81.28) (end 147.574 81.28) (width 0.25) (layer B.Cu) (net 5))
 (segment (start 147.574 81.28) (end 148.336 80.518) (width 0.25) (layer B.Cu) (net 5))
 (segment (start 149.947999 103.036001) (end 149.098 103.886) (width 0.25) (layer B.Cu) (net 5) (status 20))
 (segment (start 152.012003 102.710999) (end 150.273001 102.710999) (width 0.25) (layer B.Cu) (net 5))
 (segment (start 150.273001 102.710999) (end 149.947999 103.036001) (width 0.25) (layer B.Cu) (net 5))
 (segment (start 152.813001 101.910001) (end 152.012003 102.710999) (width 0.25) (layer B.Cu) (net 5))
 (segment (start 152.813001 81.947001) (end 152.813001 101.910001) (width 0.25) (layer B.Cu) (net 5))
 (segment (start 151.384 80.518) (end 152.813001 81.947001) (width 0.25) (layer B.Cu) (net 5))
 (segment (start 148.336 80.518) (end 151.384 80.518) (width 0.25) (layer B.Cu) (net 5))
 (segment (start 135.391 81.525) (end 135.636 81.28) (width 0.25) (layer B.Cu) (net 5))
 (segment (start 134.366 81.525) (end 135.391 81.525) (width 0.25) (layer B.Cu) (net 5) (status 10))
 (segment (start 152.651001 108.490001) (end 138.830001 108.490001) (width 0.25) (layer F.Cu) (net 5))
 (segment (start 152.716001 108.425001) (end 152.651001 108.490001) (width 0.25) (layer F.Cu) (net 5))
 (segment (start 152.716001 106.204999) (end 152.716001 108.425001) (width 0.25) (layer F.Cu) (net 5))
 (segment (start 151.572003 105.061001) (end 152.716001 106.204999) (width 0.25) (layer F.Cu) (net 5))
 (segment (start 137.655 107.315) (end 136.955 107.315) (width 0.25) (layer F.Cu) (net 5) (status 20))
 (segment (start 150.273001 105.061001) (end 151.572003 105.061001) (width 0.25) (layer F.Cu) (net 5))
 (segment (start 138.830001 108.490001) (end 137.655 107.315) (width 0.25) (layer F.Cu) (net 5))
 (segment (start 149.098 103.886) (end 150.273001 105.061001) (width 0.25) (layer F.Cu) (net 5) (status 10))
 (segment (start 146.558 100.143919) (end 146.558 101.346) (width 0.25) (layer F.Cu) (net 12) (status 20))
 (segment (start 146.877999 94.292001) (end 146.877999 99.82392) (width 0.25) (layer F.Cu) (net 12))
 (segment (start 146.877999 99.82392) (end 146.558 100.143919) (width 0.25) (layer F.Cu) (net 12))
 (segment (start 149.763 91.407) (end 146.877999 94.292001) (width 0.25) (layer F.Cu) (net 12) (status 10))
 (segment (start 147.407999 103.036001) (end 146.558 103.886) (width 0.25) (layer F.Cu) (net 6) (status 20))
 (segment (start 147.733001 102.710999) (end 147.407999 103.036001) (width 0.25) (layer F.Cu) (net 6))
 (segment (start 152.93802 101.784982) (end 152.012003 102.710999) (width 0.25) (layer F.Cu) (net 6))
 (segment (start 151.973001 80.531999) (end 152.93802 81.497018) (width 0.25) (layer F.Cu) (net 6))
 (segment (start 146.981003 80.531999) (end 151.973001 80.531999) (width 0.25) (layer F.Cu) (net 6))
 (segment (start 142.106002 85.407) (end 146.981003 80.531999) (width 0.25) (layer F.Cu) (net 6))
 (segment (start 152.012003 102.710999) (end 147.733001 102.710999) (width 0.25) (layer F.Cu) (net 6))
 (segment (start 152.93802 81.497018) (end 152.93802 101.784982) (width 0.25) (layer F.Cu) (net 6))
 (segment (start 135.763 85.407) (end 142.106002 85.407) (width 0.25) (layer F.Cu) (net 6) (status 10))
 (via (at 134.366 85.471) (size 0.8) (drill 0.4) (layers F.Cu B.Cu) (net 6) (status 30))
 (segment (start 152.488011 100.495989) (end 152.487999 100.496001) (width 0.25) (layer F.Cu) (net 16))
 (segment (start 152.487999 100.496001) (end 151.638 101.346) (width 0.25) (layer F.Cu) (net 16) (status 20))
 (segment (start 152.488011 85.047009) (end 152.488011 100.495989) (width 0.25) (layer F.Cu) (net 16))
 (segment (start 150.848002 83.407) (end 152.488011 85.047009) (width 0.25) (layer F.Cu) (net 16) (status 10))
 (segment (start 149.763 83.407) (end 150.848002 83.407) (width 0.25) (layer F.Cu) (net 16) (status 30))
 (via (at 149.606 81.534) (size 0.8) (drill 0.4) (layers F.Cu B.Cu) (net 17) (status 30))
 (segment (start 152.362991 82.385991) (end 151.511 81.534) (width 0.25) (layer B.Cu) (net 17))
 (segment (start 151.511 81.534) (end 149.606 81.534) (width 0.25) (layer B.Cu) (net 17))
 (segment (start 147.733001 101.910001) (end 147.733001 100.932999) (width 0.25) (layer B.Cu) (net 17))
 (segment (start 146.932003 102.710999) (end 147.733001 101.910001) (width 0.25) (layer B.Cu) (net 17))
 (segment (start 147.733001 100.932999) (end 152.362991 96.303009) (width 0.25) (layer B.Cu) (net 17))
 (segment (start 152.362991 96.303009) (end 152.362991 82.385991) (width 0.25) (layer B.Cu) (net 17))
 (segment (start 145.193001 102.710999) (end 146.932003 102.710999) (width 0.25) (layer B.Cu) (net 17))
 (segment (start 144.018 103.886) (end 145.193001 102.710999) (width 0.25) (layer B.Cu) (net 17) (status 10))
 (segment (start 142.842999 99.981001) (end 142.327999 100.496001) (width 0.25) (layer F.Cu) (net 15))
 (segment (start 142.327999 100.496001) (end 141.478 101.346) (width 0.25) (layer F.Cu) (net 15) (status 20))
 (segment (start 142.842999 94.641999) (end 142.842999 99.981001) (width 0.25) (layer F.Cu) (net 15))
 (segment (start 148.952999 88.531999) (end 142.842999 94.641999) (width 0.25) (layer F.Cu) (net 15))
 (segment (start 151.723003 88.531999) (end 148.952999 88.531999) (width 0.25) (layer F.Cu) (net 15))
 (segment (start 150.848002 85.407) (end 152.038001 86.596999) (width 0.25) (layer F.Cu) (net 15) (status 10))
 (segment (start 149.763 85.407) (end 150.848002 85.407) (width 0.25) (layer F.Cu) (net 15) (status 30))
 (segment (start 152.038001 88.217001) (end 151.723003 88.531999) (width 0.25) (layer F.Cu) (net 15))
 (segment (start 152.038001 86.596999) (end 152.038001 88.217001) (width 0.25) (layer F.Cu) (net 15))
 (segment (start 148.887999 86.531999) (end 149.763 87.407) (width 0.25) (layer F.Cu) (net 14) (status 20))
 (segment (start 133.552999 86.531999) (end 148.887999 86.531999) (width 0.25) (layer F.Cu) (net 14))
 (segment (start 132.43001 102.45801) (end 132.43001 87.654988) (width 0.25) (layer F.Cu) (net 14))
 (segment (start 132.43001 87.654988) (end 133.552999 86.531999) (width 0.25) (layer F.Cu) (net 14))
 (segment (start 133.858 103.886) (end 132.43001 102.45801) (width 0.25) (layer F.Cu) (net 14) (status 10))
 (via (at 149.86 93.218) (size 0.8) (drill 0.4) (layers F.Cu B.Cu) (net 11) (status 30))
 (segment (start 150.114 93.218) (end 149.86 93.472) (width 0.25) (layer B.Cu) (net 11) (status 30))
 (segment (start 150.114 93.1254) (end 150.114 93.218) (width 0.25) (layer B.Cu) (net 11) (status 30))
 (segment (start 148.16 106.934) (end 148.541 107.315) (width 0.25) (layer F.Cu) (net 2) (status 30))
 (segment (start 144.154 106.934) (end 148.16 106.934) (width 0.25) (layer F.Cu) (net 2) (status 30)))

